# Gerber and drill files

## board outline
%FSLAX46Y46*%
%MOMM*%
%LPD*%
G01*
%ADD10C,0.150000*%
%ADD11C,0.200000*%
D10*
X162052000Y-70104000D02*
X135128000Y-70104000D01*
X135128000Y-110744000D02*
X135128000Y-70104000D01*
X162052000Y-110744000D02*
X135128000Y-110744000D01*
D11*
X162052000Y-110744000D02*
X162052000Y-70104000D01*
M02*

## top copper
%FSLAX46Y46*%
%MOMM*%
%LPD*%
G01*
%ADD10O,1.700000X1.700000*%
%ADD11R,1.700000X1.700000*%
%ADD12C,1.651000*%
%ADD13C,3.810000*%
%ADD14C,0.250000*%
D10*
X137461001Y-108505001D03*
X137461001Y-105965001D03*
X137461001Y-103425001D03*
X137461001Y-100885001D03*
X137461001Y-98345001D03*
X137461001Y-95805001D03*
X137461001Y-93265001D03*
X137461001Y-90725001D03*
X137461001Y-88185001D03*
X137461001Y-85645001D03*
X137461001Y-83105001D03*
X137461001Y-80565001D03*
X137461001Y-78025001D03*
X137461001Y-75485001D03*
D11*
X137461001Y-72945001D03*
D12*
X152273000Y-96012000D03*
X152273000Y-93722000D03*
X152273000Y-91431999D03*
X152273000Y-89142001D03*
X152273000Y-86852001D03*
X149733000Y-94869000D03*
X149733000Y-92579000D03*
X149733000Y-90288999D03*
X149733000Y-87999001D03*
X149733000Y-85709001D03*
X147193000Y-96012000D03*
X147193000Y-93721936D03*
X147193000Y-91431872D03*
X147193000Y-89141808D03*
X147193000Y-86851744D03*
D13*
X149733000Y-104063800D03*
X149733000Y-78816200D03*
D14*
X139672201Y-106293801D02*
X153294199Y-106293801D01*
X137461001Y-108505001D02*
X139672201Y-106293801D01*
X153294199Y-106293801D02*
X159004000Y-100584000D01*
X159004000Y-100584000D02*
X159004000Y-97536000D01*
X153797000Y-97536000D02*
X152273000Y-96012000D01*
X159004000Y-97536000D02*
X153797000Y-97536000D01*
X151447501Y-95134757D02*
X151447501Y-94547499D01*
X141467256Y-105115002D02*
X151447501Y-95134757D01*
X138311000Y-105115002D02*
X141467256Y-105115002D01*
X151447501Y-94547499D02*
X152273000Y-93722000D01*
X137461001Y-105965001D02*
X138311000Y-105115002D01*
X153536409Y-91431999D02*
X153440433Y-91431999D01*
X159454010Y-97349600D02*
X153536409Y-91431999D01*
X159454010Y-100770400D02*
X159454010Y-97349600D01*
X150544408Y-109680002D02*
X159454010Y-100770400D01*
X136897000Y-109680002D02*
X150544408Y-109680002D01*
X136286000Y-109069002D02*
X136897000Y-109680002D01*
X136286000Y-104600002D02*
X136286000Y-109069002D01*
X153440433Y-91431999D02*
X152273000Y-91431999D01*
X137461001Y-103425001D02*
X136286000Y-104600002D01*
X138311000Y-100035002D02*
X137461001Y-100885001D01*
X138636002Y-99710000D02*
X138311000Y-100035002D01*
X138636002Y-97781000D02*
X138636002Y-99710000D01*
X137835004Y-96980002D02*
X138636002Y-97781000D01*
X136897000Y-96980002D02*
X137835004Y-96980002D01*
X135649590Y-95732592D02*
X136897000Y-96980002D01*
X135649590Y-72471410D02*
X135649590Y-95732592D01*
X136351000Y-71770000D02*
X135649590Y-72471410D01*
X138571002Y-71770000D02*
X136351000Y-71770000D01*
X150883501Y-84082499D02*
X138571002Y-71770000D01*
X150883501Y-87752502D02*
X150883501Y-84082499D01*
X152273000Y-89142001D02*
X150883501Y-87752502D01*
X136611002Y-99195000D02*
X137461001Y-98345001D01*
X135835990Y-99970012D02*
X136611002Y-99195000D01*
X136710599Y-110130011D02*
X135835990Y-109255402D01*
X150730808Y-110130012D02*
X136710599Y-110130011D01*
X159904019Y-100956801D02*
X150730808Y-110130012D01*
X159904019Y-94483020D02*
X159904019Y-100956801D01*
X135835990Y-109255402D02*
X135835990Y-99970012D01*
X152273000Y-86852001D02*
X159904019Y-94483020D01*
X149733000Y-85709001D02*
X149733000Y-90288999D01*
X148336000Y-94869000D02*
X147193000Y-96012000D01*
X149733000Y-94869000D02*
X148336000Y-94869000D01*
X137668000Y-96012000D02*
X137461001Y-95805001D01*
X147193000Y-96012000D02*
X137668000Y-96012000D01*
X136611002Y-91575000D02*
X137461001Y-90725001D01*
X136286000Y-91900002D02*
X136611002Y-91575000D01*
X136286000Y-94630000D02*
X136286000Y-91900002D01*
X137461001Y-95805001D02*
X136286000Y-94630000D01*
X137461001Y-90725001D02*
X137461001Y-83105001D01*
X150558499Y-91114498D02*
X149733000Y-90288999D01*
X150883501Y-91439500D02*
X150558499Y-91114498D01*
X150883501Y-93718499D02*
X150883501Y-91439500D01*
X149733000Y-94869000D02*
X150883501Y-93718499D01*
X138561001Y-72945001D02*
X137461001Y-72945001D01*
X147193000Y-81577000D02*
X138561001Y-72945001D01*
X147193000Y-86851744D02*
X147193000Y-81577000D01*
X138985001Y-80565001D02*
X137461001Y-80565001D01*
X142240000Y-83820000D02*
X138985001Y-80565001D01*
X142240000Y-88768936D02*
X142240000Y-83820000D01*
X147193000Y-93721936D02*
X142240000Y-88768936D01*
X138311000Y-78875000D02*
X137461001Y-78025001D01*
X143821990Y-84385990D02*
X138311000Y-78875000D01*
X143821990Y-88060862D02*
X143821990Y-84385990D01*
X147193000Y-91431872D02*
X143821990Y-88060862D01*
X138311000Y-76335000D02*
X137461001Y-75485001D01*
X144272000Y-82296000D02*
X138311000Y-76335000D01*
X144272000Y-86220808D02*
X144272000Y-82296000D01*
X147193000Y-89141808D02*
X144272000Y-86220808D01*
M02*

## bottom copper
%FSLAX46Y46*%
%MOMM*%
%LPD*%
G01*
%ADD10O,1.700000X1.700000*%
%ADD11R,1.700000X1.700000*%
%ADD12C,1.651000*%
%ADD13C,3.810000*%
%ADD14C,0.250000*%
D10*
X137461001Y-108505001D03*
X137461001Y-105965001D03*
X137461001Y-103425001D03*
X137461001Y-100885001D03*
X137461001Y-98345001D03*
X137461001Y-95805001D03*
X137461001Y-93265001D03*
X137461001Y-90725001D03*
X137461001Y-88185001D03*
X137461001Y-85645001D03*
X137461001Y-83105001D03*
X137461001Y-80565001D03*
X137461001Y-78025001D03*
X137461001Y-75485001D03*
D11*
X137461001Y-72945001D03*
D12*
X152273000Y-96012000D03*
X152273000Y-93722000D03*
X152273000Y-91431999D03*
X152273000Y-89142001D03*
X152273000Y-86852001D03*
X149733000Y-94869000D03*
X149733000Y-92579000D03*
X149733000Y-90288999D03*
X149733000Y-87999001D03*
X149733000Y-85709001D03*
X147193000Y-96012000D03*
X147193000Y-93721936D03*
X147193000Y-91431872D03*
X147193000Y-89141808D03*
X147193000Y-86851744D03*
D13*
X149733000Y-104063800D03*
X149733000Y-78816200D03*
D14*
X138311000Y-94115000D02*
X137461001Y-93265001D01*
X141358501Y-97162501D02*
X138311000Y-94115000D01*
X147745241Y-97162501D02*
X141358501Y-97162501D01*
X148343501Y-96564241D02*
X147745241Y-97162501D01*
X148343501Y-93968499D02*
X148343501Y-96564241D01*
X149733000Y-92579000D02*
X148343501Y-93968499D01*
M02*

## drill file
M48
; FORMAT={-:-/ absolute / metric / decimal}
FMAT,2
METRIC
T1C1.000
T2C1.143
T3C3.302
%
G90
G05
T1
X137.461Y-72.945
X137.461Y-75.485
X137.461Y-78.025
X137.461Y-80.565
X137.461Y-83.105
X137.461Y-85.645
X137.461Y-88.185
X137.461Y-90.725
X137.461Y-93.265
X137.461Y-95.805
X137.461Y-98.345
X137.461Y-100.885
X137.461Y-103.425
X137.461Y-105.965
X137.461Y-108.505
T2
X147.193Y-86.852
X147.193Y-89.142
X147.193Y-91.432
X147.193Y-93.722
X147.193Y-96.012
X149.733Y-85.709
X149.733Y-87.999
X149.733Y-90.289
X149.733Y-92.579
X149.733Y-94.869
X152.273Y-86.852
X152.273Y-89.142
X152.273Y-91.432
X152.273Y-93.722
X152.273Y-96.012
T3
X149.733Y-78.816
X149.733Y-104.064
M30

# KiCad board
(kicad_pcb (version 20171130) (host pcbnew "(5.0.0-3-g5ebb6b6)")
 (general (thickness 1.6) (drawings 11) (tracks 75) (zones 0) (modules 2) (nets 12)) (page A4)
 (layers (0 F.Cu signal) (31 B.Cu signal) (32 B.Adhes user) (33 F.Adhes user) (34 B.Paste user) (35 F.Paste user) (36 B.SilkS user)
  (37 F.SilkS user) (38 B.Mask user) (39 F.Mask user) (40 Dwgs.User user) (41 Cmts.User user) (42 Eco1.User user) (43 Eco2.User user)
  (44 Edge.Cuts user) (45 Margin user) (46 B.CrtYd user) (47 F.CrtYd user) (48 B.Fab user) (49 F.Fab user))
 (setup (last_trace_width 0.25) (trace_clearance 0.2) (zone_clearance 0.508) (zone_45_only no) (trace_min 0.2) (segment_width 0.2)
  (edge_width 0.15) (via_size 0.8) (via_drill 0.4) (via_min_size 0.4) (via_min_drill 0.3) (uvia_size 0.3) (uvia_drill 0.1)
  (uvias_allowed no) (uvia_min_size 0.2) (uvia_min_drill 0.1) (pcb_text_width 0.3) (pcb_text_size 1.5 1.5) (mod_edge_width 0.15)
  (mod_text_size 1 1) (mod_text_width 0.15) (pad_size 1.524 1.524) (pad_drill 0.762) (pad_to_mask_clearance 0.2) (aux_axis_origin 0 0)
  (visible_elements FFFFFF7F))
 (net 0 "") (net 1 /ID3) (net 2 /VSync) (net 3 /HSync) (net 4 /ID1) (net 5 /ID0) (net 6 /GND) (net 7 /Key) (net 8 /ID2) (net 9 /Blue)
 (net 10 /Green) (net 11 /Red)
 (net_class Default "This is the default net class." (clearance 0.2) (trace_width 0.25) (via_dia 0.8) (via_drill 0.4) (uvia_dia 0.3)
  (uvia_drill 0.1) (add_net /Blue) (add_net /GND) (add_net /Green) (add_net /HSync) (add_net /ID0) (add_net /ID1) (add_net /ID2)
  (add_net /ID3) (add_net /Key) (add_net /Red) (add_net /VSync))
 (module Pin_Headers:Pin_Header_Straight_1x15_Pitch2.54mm (layer F.Cu) (at 137.461001 72.945001)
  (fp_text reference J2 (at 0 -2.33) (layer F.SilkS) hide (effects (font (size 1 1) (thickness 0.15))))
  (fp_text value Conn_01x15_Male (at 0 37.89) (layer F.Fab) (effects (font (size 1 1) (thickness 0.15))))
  (pad 15 thru_hole oval (at 0 35.56) (size 1.7 1.7) (drill 1) (layers *.Cu *.Mask) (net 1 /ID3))
  (pad 14 thru_hole oval (at 0 33.02) (size 1.7 1.7) (drill 1) (layers *.Cu *.Mask) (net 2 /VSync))
  (pad 13 thru_hole oval (at 0 30.48) (size 1.7 1.7) (drill 1) (layers *.Cu *.Mask) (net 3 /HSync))
  (pad 12 thru_hole oval (at 0 27.94) (size 1.7 1.7) (drill 1) (layers *.Cu *.Mask) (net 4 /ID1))
  (pad 11 thru_hole oval (at 0 25.4) (size 1.7 1.7) (drill 1) (layers *.Cu *.Mask) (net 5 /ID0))
  (pad 10 thru_hole oval (at 0 22.86) (size 1.7 1.7) (drill 1) (layers *.Cu *.Mask) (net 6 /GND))
  (pad 9 thru_hole oval (at 0 20.32) (size 1.7 1.7) (drill 1) (layers *.Cu *.Mask) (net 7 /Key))
  (pad 8 thru_hole oval (at 0 17.78) (size 1.7 1.7) (drill 1) (layers *.Cu *.Mask) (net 6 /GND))
  (pad 7 thru_hole oval (at 0 15.24) (size 1.7 1.7) (drill 1) (layers *.Cu *.Mask) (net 6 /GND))
  (pad 6 thru_hole oval (at 0 12.7) (size 1.7 1.7) (drill 1) (layers *.Cu *.Mask) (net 6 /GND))
  (pad 5 thru_hole oval (at 0 10.16) (size 1.7 1.7) (drill 1) (layers *.Cu *.Mask) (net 6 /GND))
  (pad 4 thru_hole oval (at 0 7.62) (size 1.7 1.7) (drill 1) (layers *.Cu *.Mask) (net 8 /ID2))
  (pad 3 thru_hole oval (at 0 5.08) (size 1.7 1.7) (drill 1) (layers *.Cu *.Mask) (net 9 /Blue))
  (pad 2 thru_hole oval (at 0 2.54) (size 1.7 1.7) (drill 1) (layers *.Cu *.Mask) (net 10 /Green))
  (pad 1 thru_hole rect (at 0 0) (size 1.7 1.7) (drill 1) (layers *.Cu *.Mask) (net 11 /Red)))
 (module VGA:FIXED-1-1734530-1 (layer F.Cu) (at 161.544 91.44 270)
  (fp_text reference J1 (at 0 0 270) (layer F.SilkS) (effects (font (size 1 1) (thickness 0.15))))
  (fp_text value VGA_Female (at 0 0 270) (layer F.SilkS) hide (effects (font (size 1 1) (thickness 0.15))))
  (pad 15 thru_hole circle (at 4.572 9.271 270) (size 1.651 1.651) (drill 1.143) (layers *.Cu *.Mask) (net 1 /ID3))
  (pad 14 thru_hole circle (at 2.282 9.271 270) (size 1.651 1.651) (drill 1.143) (layers *.Cu *.Mask) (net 2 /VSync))
  (pad 13 thru_hole circle (at -0.008001 9.271 270) (size 1.651 1.651) (drill 1.143) (layers *.Cu *.Mask) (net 3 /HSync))
  (pad 12 thru_hole circle (at -2.297999 9.271 270) (size 1.651 1.651) (drill 1.143) (layers *.Cu *.Mask) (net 4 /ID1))
  (pad 11 thru_hole circle (at -4.587999 9.271 270) (size 1.651 1.651) (drill 1.143) (layers *.Cu *.Mask) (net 5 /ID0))
  (pad 10 thru_hole circle (at 3.429 11.811 270) (size 1.651 1.651) (drill 1.143) (layers *.Cu *.Mask) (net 6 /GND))
  (pad 9 thru_hole circle (at 1.139 11.811 270) (size 1.651 1.651) (drill 1.143) (layers *.Cu *.Mask) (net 7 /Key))
  (pad 8 thru_hole circle (at -1.151001 11.811 270) (size 1.651 1.651) (drill 1.143) (layers *.Cu *.Mask) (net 6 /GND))
  (pad 7 thru_hole circle (at -3.440999 11.811 270) (size 1.651 1.651) (drill 1.143) (layers *.Cu *.Mask) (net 6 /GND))
  (pad 6 thru_hole circle (at -5.730999 11.811 270) (size 1.651 1.651) (drill 1.143) (layers *.Cu *.Mask) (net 6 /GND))
  (pad 5 thru_hole circle (at 4.572 14.351 270) (size 1.651 1.651) (drill 1.143) (layers *.Cu *.Mask) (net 6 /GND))
  (pad 4 thru_hole circle (at 2.281936 14.351 270) (size 1.651 1.651) (drill 1.143) (layers *.Cu *.Mask) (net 8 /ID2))
  (pad 3 thru_hole circle (at -0.008128 14.351 270) (size 1.651 1.651) (drill 1.143) (layers *.Cu *.Mask) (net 9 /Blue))
  (pad 2 thru_hole circle (at -2.298192 14.351 270) (size 1.651 1.651) (drill 1.143) (layers *.Cu *.Mask) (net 10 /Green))
  (pad 1 thru_hole circle (at -4.588256 14.351 270) (size 1.651 1.651) (drill 1.143) (layers *.Cu *.Mask) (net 11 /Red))
  (pad 16 thru_hole circle (at 12.6238 11.811 270) (size 3.81 3.81) (drill 3.302) (layers *.Cu *.Mask))
  (pad 17 thru_hole circle (at -12.6238 11.811 270) (size 3.81 3.81) (drill 3.302) (layers *.Cu *.Mask)))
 (gr_line (start 162.052 70.104) (end 135.128 70.104) (layer Edge.Cuts) (width 0.15))
 (gr_line (start 135.128 110.744) (end 135.128 70.104) (layer Edge.Cuts) (width 0.15))
 (gr_line (start 162.052 110.744) (end 135.128 110.744) (layer Edge.Cuts) (width 0.15))
 (gr_line (start 162.052 110.744) (end 162.052 70.104) (layer Edge.Cuts) (width 0.2))
 (segment (start 139.672201 106.293801) (end 153.294199 106.293801) (width 0.25) (layer F.Cu) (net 1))
 (segment (start 137.461001 108.505001) (end 139.672201 106.293801) (width 0.25) (layer F.Cu) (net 1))
 (segment (start 153.294199 106.293801) (end 159.004 100.584) (width 0.25) (layer F.Cu) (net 1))
 (segment (start 159.004 100.584) (end 159.004 97.536) (width 0.25) (layer F.Cu) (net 1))
 (segment (start 153.797 97.536) (end 152.273 96.012) (width 0.25) (layer F.Cu) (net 1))
 (segment (start 159.004 97.536) (end 153.797 97.536) (width 0.25) (layer F.Cu) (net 1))
 (segment (start 151.447501 95.134757) (end 151.447501 94.547499) (width 0.25) (layer F.Cu) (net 2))
 (segment (start 141.467256 105.115002) (end 151.447501 95.134757) (width 0.25) (layer F.Cu) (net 2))
 (segment (start 138.311 105.115002) (end 141.467256 105.115002) (width 0.25) (layer F.Cu) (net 2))
 (segment (start 151.447501 94.547499) (end 152.273 93.722) (width 0.25) (layer F.Cu) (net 2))
 (segment (start 137.461001 105.965001) (end 138.311 105.115002) (width 0.25) (layer F.Cu) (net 2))
 (segment (start 153.536409 91.431999) (end 153.440433 91.431999) (width 0.25) (layer F.Cu) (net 3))
 (segment (start 159.45401 97.3496) (end 153.536409 91.431999) (width 0.25) (layer F.Cu) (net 3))
 (segment (start 159.45401 100.7704) (end 159.45401 97.3496) (width 0.25) (layer F.Cu) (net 3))
 (segment (start 150.544408 109.680002) (end 159.45401 100.7704) (width 0.25) (layer F.Cu) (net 3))
 (segment (start 136.897 109.680002) (end 150.544408 109.680002) (width 0.25) (layer F.Cu) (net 3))
 (segment (start 136.286 109.069002) (end 136.897 109.680002) (width 0.25) (layer F.Cu) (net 3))
 (segment (start 136.286 104.600002) (end 136.286 109.069002) (width 0.25) (layer F.Cu) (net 3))
 (segment (start 153.440433 91.431999) (end 152.273 91.431999) (width 0.25) (layer F.Cu) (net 3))
 (segment (start 137.461001 103.425001) (end 136.286 104.600002) (width 0.25) (layer F.Cu) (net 3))
 (segment (start 138.311 100.035002) (end 137.461001 100.885001) (width 0.25) (layer F.Cu) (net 4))
 (segment (start 138.636002 99.71) (end 138.311 100.035002) (width 0.25) (layer F.Cu) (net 4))
 (segment (start 138.636002 97.781) (end 138.636002 99.71) (width 0.25) (layer F.Cu) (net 4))
 (segment (start 137.835004 96.980002) (end 138.636002 97.781) (width 0.25) (layer F.Cu) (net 4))
 (segment (start 136.897 96.980002) (end 137.835004 96.980002) (width 0.25) (layer F.Cu) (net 4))
 (segment (start 135.64959 95.732592) (end 136.897 96.980002) (width 0.25) (layer F.Cu) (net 4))
 (segment (start 135.64959 72.47141) (end 135.64959 95.732592) (width 0.25) (layer F.Cu) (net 4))
 (segment (start 136.351 71.77) (end 135.64959 72.47141) (width 0.25) (layer F.Cu) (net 4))
 (segment (start 138.571002 71.77) (end 136.351 71.77) (width 0.25) (layer F.Cu) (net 4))
 (segment (start 150.883501 84.082499) (end 138.571002 71.77) (width 0.25) (layer F.Cu) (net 4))
 (segment (start 150.883501 87.752502) (end 150.883501 84.082499) (width 0.25) (layer F.Cu) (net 4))
 (segment (start 152.273 89.142001) (end 150.883501 87.752502) (width 0.25) (layer F.Cu) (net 4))
 (segment (start 136.611002 99.195) (end 137.461001 98.345001) (width 0.25) (layer F.Cu) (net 5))
 (segment (start 135.83599 99.970012) (end 136.611002 99.195) (width 0.25) (layer F.Cu) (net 5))
 (segment (start 136.710599 110.130011) (end 135.83599 109.255402) (width 0.25) (layer F.Cu) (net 5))
 (segment (start 150.730808 110.130012) (end 136.710599 110.130011) (width 0.25) (layer F.Cu) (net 5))
 (segment (start 159.904019 100.956801) (end 150.730808 110.130012) (width 0.25) (layer F.Cu) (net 5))
 (segment (start 159.904019 94.48302) (end 159.904019 100.956801) (width 0.25) (layer F.Cu) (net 5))
 (segment (start 135.83599 109.255402) (end 135.83599 99.970012) (width 0.25) (layer F.Cu) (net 5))
 (segment (start 152.273 86.852001) (end 159.904019 94.48302) (width 0.25) (layer F.Cu) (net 5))
 (segment (start 149.733 85.709001) (end 149.733 90.288999) (width 0.25) (layer F.Cu) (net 6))
 (segment (start 148.336 94.869) (end 147.193 96.012) (width 0.25) (layer F.Cu) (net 6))
 (segment (start 149.733 94.869) (end 148.336 94.869) (width 0.25) (layer F.Cu) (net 6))
 (segment (start 137.668 96.012) (end 137.461001 95.805001) (width 0.25) (layer F.Cu) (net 6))
 (segment (start 147.193 96.012) (end 137.668 96.012) (width 0.25) (layer F.Cu) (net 6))
 (segment (start 136.611002 91.575) (end 137.461001 90.725001) (width 0.25) (layer F.Cu) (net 6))
 (segment (start 136.286 91.900002) (end 136.611002 91.575) (width 0.25) (layer F.Cu) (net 6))
 (segment (start 136.286 94.63) (end 136.286 91.900002) (width 0.25) (layer F.Cu) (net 6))
 (segment (start 137.461001 95.805001) (end 136.286 94.63) (width 0.25) (layer F.Cu) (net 6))
 (segment (start 137.461001 90.725001) (end 137.461001 83.105001) (width 0.25) (layer F.Cu) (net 6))
 (segment (start 150.558499 91.114498) (end 149.733 90.288999) (width 0.25) (layer F.Cu) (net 6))
 (segment (start 150.883501 91.4395) (end 150.558499 91.114498) (width 0.25) (layer F.Cu) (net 6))
 (segment (start 150.883501 93.718499) (end 150.883501 91.4395) (width 0.25) (layer F.Cu) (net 6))
 (segment (start 149.733 94.869) (end 150.883501 93.718499) (width 0.25) (layer F.Cu) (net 6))
 (segment (start 138.311 94.115) (end 137.461001 93.265001) (width 0.25) (layer B.Cu) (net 7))
 (segment (start 141.358501 97.162501) (end 138.311 94.115) (width 0.25) (layer B.Cu) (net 7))
 (segment (start 147.745241 97.162501) (end 141.358501 97.162501) (width 0.25) (layer B.Cu) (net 7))
 (segment (start 148.343501 96.564241) (end 147.745241 97.162501) (width 0.25) (layer B.Cu) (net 7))
 (segment (start 148.343501 93.968499) (end 148.343501 96.564241) (width 0.25) (layer B.Cu) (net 7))
 (segment (start 149.733 92.579) (end 148.343501 93.968499) (width 0.25) (layer B.Cu) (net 7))
 (segment (start 138.561001 72.945001) (end 137.461001 72.945001) (width 0.25) (layer F.Cu) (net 11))
 (segment (start 147.193 81.577) (end 138.561001 72.945001) (width 0.25) (layer F.Cu) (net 11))
 (segment (start 147.193 86.851744) (end 147.193 81.577) (width 0.25) (layer F.Cu) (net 11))
 (segment (start 138.985001 80.565001) (end 137.461001 80.565001) (width 0.25) (layer F.Cu) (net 8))
 (segment (start 142.24 83.82) (end 138.985001 80.565001) (width 0.25) (layer F.Cu) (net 8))
 (segment (start 142.24 88.768936) (end 142.24 83.82) (width 0.25) (layer F.Cu) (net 8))
 (segment (start 147.193 93.721936) (end 142.24 88.768936) (width 0.25) (layer F.Cu) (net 8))
 (segment (start 138.311 78.875) (end 137.461001 78.025001) (width 0.25) (layer F.Cu) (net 9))
 (segment (start 143.82199 84.38599) (end 138.311 78.875) (width 0.25) (layer F.Cu) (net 9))
 (segment (start 143.82199 88.060862) (end 143.82199 84.38599) (width 0.25) (layer F.Cu) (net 9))
 (segment (start 147.193 91.431872) (end 143.82199 88.060862) (width 0.25) (layer F.Cu) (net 9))
 (segment (start 138.311 76.335) (end 137.461001 75.485001) (width 0.25) (layer F.Cu) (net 10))
 (segment (start 144.272 82.296) (end 138.311 76.335) (width 0.25) (layer F.Cu) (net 10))
 (segment (start 144.272 86.220808) (end 144.272 82.296) (width 0.25) (layer F.Cu) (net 10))
 (segment (start 147.193 89.141808) (end 144.272 86.220808) (width 0.25) (layer F.Cu) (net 10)))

